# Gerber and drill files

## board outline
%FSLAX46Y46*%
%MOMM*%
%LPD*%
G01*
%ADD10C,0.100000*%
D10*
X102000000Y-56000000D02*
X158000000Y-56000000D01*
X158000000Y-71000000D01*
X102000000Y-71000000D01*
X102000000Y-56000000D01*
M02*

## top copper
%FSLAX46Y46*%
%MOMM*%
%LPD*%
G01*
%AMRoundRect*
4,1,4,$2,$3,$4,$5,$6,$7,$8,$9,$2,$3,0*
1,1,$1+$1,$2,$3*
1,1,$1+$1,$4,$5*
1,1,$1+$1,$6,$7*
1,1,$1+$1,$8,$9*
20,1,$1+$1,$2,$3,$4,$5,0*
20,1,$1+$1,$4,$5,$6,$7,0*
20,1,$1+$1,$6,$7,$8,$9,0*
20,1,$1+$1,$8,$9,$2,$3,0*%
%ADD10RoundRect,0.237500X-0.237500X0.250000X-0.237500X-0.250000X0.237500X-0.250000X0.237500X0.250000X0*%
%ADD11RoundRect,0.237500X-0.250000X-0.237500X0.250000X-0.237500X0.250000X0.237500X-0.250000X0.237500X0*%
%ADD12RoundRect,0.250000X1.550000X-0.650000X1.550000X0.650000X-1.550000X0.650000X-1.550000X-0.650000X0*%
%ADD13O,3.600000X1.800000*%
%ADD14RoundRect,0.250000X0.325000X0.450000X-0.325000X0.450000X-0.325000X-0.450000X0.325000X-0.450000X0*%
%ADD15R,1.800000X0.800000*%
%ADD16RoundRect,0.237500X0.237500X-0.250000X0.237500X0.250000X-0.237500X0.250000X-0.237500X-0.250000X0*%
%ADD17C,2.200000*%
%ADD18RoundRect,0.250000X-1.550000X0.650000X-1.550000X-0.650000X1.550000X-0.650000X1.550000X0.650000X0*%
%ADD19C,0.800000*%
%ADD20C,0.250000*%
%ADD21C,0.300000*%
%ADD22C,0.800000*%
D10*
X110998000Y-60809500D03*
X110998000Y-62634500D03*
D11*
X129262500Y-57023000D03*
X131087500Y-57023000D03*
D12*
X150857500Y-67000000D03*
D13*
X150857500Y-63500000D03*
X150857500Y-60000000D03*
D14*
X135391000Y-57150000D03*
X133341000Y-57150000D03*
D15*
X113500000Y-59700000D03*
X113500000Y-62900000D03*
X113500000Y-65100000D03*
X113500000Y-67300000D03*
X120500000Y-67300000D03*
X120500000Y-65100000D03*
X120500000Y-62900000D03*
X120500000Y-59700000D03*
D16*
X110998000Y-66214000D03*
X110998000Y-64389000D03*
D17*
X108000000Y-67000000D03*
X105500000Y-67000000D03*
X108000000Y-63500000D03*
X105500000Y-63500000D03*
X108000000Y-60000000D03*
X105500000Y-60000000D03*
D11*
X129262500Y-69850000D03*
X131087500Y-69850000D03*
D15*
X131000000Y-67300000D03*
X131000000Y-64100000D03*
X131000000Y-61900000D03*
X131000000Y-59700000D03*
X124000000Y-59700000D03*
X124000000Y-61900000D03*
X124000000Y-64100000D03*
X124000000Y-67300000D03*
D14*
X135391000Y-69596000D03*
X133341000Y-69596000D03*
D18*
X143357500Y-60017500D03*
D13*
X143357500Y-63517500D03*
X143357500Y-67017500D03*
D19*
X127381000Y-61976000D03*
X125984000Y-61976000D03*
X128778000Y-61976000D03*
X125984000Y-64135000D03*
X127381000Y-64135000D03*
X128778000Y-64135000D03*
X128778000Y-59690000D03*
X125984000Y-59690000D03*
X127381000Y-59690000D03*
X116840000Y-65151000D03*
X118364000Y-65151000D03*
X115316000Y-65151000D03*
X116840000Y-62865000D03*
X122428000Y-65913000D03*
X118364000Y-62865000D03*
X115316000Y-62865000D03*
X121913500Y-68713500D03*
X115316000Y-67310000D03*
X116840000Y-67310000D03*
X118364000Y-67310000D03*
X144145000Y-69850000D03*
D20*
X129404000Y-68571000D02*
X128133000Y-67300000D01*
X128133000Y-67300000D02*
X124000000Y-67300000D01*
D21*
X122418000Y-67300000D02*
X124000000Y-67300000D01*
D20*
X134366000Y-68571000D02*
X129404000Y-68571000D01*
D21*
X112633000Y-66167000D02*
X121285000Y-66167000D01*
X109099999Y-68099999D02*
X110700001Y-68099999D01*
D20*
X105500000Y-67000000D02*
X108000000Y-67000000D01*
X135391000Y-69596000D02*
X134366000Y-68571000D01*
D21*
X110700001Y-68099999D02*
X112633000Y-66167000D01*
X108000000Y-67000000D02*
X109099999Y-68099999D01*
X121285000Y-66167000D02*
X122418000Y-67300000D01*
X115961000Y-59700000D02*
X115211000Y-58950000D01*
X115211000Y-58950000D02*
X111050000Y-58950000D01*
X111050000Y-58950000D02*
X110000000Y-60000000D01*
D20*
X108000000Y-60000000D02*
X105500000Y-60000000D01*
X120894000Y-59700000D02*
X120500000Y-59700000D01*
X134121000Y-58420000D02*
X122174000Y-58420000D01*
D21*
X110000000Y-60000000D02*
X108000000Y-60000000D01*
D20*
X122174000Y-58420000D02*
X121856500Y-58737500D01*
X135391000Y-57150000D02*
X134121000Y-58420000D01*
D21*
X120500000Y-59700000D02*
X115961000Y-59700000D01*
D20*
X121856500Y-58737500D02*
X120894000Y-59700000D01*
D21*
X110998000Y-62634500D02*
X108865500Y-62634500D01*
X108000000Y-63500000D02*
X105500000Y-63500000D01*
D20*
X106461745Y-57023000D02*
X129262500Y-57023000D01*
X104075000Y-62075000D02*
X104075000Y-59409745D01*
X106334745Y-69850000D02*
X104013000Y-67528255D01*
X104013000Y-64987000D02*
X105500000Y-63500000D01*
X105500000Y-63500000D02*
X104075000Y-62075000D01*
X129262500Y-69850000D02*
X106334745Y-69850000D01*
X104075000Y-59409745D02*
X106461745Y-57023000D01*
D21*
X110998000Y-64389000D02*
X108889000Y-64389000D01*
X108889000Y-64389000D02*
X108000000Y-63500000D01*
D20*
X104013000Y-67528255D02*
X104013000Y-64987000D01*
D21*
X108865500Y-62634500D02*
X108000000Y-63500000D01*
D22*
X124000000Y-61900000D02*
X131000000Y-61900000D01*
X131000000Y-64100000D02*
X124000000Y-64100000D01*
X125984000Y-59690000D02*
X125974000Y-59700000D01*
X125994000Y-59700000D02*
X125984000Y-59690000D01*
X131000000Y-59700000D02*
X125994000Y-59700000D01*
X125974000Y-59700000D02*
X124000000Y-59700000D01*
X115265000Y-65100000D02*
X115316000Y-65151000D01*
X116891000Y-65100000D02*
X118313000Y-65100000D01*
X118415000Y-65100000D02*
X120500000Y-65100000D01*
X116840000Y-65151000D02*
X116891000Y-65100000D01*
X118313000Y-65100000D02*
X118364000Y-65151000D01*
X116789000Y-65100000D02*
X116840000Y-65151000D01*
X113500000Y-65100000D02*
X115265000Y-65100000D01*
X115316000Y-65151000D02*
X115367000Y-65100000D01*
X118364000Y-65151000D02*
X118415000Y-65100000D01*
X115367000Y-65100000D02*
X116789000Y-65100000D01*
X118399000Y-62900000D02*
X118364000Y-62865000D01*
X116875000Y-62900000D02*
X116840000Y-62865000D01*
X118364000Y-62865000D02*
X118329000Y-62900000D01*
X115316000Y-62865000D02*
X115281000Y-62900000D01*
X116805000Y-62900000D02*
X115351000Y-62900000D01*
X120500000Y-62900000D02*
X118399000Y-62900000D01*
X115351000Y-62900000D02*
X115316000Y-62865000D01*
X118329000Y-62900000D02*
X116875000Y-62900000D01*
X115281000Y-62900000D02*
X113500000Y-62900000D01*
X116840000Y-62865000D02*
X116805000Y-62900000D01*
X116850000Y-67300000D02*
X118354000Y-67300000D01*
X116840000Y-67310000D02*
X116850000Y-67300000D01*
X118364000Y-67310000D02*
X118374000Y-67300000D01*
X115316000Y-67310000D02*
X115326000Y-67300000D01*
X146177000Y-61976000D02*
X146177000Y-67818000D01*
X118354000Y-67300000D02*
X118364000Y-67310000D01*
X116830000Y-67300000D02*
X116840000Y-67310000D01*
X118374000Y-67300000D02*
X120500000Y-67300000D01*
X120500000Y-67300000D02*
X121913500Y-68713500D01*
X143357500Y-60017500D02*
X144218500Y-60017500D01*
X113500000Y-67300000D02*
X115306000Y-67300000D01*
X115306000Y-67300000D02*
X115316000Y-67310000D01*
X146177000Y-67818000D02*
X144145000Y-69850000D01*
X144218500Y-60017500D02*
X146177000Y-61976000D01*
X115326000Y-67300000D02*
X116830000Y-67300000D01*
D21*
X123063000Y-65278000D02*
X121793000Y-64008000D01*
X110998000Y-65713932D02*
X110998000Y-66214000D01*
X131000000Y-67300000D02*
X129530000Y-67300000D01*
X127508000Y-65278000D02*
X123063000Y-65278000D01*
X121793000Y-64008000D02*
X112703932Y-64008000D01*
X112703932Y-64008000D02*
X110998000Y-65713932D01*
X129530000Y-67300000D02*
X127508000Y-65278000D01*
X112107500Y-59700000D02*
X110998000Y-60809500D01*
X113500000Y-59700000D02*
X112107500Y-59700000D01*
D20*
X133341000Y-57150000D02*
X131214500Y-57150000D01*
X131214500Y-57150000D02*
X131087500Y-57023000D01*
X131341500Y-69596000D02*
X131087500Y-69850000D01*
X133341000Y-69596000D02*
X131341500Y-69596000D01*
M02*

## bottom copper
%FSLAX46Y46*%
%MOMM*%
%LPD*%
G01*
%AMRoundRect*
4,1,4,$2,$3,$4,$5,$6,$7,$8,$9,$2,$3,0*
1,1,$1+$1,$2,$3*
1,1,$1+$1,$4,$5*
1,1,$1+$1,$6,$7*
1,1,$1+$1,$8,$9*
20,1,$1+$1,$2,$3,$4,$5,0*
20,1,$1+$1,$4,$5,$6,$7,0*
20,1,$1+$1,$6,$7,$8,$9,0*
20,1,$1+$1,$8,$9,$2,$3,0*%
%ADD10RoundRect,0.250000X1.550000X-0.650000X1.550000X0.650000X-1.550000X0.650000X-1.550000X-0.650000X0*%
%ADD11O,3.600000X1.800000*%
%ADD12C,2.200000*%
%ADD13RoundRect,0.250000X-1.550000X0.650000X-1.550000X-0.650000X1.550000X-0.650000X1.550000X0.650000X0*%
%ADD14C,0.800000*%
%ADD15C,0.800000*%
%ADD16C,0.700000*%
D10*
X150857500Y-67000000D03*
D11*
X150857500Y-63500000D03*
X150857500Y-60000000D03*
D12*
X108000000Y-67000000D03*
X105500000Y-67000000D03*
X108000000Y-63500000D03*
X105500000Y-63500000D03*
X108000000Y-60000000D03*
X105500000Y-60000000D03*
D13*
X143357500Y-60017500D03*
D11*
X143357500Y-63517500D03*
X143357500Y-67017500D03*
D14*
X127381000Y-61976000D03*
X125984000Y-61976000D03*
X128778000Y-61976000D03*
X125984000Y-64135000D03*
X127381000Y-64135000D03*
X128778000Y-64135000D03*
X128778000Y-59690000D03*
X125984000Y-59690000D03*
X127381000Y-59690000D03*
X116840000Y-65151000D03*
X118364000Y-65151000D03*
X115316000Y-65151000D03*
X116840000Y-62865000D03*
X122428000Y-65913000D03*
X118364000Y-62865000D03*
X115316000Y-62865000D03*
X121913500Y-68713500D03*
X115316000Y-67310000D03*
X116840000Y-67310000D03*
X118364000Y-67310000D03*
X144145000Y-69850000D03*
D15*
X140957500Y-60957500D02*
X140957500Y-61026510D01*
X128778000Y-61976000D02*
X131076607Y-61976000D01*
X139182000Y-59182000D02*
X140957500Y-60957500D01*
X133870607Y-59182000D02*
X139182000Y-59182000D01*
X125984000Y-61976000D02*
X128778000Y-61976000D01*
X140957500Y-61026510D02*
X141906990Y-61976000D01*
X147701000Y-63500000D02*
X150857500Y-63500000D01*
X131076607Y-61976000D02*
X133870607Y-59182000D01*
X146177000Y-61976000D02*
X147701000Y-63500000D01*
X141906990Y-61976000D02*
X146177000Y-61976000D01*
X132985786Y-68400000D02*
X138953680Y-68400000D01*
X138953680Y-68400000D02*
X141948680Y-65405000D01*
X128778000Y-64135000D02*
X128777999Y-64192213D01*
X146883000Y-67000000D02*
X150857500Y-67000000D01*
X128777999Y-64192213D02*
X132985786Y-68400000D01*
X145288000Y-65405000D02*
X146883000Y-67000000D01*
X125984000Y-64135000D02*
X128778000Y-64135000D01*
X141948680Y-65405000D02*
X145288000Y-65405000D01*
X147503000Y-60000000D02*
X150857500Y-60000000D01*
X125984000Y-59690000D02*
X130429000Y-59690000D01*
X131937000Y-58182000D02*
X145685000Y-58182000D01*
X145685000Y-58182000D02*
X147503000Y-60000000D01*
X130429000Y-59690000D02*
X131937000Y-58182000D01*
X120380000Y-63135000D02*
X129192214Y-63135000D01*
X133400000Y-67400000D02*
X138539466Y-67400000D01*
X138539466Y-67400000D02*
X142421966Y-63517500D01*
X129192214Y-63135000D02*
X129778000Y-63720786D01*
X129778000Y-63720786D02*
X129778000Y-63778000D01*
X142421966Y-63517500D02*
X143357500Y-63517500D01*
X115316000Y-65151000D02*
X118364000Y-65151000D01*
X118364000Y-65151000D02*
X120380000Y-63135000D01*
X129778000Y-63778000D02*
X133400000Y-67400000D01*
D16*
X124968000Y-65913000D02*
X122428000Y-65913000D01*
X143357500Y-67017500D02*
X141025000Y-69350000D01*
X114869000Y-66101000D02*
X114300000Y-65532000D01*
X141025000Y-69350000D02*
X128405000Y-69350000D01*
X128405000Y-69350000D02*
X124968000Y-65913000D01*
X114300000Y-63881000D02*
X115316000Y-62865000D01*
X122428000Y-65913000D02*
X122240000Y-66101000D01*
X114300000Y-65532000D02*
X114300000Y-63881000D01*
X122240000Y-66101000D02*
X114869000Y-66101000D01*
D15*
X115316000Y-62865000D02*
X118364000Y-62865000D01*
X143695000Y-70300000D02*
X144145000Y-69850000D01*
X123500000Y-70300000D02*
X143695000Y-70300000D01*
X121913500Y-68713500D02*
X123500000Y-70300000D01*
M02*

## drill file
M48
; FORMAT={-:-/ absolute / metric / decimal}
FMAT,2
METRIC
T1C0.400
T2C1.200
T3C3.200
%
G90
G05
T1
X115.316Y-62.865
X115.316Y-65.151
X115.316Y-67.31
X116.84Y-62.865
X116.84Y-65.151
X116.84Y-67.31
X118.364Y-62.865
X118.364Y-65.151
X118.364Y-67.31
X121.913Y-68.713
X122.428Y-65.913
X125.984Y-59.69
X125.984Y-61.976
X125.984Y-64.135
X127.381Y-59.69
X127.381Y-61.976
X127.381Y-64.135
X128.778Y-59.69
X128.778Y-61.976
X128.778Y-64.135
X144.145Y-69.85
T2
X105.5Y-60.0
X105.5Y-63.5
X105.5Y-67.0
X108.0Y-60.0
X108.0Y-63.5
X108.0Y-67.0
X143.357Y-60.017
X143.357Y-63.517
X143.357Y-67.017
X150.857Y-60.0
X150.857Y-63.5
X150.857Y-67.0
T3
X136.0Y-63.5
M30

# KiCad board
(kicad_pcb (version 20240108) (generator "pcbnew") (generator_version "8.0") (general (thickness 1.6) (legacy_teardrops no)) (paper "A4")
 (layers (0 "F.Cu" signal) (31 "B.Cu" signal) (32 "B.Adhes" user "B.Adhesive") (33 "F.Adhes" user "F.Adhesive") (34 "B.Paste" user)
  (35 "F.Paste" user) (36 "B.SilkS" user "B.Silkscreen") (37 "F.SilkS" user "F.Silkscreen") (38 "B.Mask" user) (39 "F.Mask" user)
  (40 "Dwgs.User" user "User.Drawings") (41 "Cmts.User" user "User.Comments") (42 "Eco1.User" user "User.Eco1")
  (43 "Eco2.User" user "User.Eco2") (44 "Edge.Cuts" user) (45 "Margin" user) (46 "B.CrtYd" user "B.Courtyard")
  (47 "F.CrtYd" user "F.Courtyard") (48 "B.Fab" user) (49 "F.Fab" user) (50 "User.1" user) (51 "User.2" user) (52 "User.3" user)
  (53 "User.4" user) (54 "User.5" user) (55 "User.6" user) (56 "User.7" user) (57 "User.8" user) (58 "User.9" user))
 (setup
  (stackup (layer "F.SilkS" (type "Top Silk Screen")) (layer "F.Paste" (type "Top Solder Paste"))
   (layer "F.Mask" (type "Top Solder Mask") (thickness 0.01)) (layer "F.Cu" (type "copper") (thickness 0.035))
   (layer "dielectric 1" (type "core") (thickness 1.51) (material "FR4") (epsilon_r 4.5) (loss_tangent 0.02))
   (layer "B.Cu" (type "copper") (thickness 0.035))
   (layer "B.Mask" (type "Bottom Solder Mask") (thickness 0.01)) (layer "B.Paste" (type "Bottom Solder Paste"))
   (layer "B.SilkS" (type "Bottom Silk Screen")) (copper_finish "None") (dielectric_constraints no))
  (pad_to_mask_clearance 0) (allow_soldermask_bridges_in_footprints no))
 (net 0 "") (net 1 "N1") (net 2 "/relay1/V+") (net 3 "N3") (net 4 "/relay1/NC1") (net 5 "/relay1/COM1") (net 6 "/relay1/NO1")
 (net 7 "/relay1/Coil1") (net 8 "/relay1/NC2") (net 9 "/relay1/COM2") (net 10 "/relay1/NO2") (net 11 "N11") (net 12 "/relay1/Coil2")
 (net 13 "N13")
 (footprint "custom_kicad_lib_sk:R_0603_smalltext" (layer "F.Cu") (at 110.998 61.722 -90)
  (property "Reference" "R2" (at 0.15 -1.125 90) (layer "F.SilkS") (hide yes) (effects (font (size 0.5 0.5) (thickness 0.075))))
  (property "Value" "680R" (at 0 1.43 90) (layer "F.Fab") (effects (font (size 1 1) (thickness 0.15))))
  (pad "1" smd roundrect (at -0.9125 0 270) (size 0.975 0.95) (layers "F.Cu" "F.Paste" "F.Mask") (roundrect_rratio 0.25) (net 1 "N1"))
  (pad "2" smd roundrect (at 0.9125 0 270) (size 0.975 0.95) (layers "F.Cu" "F.Paste" "F.Mask") (roundrect_rratio 0.25) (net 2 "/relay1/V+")))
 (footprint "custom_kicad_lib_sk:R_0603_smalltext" (layer "F.Cu") (at 130.175 57.023)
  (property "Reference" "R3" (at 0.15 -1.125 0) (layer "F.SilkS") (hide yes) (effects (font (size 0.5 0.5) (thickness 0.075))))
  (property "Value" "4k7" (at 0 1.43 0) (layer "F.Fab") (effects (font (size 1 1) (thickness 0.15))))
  (pad "1" smd roundrect (at -0.9125 0) (size 0.975 0.95) (layers "F.Cu" "F.Paste" "F.Mask") (roundrect_rratio 0.25) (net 2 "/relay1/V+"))
  (pad "2" smd roundrect (at 0.9125 0) (size 0.975 0.95) (layers "F.Cu" "F.Paste" "F.Mask") (roundrect_rratio 0.25) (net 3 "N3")))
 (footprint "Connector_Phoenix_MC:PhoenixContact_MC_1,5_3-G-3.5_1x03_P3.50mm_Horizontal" (layer "F.Cu") (at 150.8575 67 90)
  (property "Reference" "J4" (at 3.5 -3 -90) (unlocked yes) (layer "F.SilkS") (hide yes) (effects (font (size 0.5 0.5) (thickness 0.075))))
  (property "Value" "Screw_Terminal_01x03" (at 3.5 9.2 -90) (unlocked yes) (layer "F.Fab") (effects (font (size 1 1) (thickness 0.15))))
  (pad "1" thru_hole roundrect (at 0 0 90) (size 1.8 3.6) (drill 1.2) (layers "*.Cu" "*.Mask") (remove_unused_layers no)
   (roundrect_rratio 0.138889) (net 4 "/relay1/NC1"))
  (pad "2" thru_hole oval (at 3.5 0 90) (size 1.8 3.6) (drill 1.2) (layers "*.Cu" "*.Mask") (remove_unused_layers no) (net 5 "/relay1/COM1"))
  (pad "3" thru_hole oval (at 7 0 90) (size 1.8 3.6) (drill 1.2) (layers "*.Cu" "*.Mask") (remove_unused_layers no) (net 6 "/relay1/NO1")))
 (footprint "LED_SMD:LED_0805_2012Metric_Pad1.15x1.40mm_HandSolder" (layer "F.Cu") (at 134.366 57.15 180)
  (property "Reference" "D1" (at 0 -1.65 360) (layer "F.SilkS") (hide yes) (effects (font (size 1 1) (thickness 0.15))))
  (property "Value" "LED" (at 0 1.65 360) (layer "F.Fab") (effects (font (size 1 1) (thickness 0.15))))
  (pad "1" smd roundrect (at -1.025 0 180) (size 1.15 1.4) (layers "F.Cu" "F.Paste" "F.Mask") (roundrect_rratio 0.217391)
   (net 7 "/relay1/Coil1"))
  (pad "2" smd roundrect (at 1.025 0 180) (size 1.15 1.4) (layers "F.Cu" "F.Paste" "F.Mask") (roundrect_rratio 0.217391) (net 3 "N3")))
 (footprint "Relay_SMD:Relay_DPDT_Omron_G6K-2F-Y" (layer "F.Cu") (at 117 63.5)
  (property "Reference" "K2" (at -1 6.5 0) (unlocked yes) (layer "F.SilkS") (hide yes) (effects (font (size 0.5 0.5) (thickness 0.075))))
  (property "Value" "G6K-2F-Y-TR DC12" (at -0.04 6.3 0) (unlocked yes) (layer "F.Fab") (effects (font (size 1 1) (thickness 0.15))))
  (pad "1" smd rect (at -3.5 -3.8) (size 1.8 0.8) (layers "F.Cu" "F.Paste" "F.Mask") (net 1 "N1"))
  (pad "2" smd rect (at -3.5 -0.6) (size 1.8 0.8) (layers "F.Cu" "F.Paste" "F.Mask") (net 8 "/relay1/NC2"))
  (pad "3" smd rect (at -3.5 1.6) (size 1.8 0.8) (layers "F.Cu" "F.Paste" "F.Mask") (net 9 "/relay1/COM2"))
  (pad "4" smd rect (at -3.5 3.8) (size 1.8 0.8) (layers "F.Cu" "F.Paste" "F.Mask") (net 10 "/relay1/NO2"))
  (pad "5" smd rect (at 3.5 3.8) (size 1.8 0.8) (layers "F.Cu" "F.Paste" "F.Mask") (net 10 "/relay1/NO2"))
  (pad "6" smd rect (at 3.5 1.6) (size 1.8 0.8) (layers "F.Cu" "F.Paste" "F.Mask") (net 9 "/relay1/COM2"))
  (pad "7" smd rect (at 3.5 -0.6) (size 1.8 0.8) (layers "F.Cu" "F.Paste" "F.Mask") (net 8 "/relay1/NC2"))
  (pad "8" smd rect (at 3.5 -3.8) (size 1.8 0.8) (layers "F.Cu" "F.Paste" "F.Mask") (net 7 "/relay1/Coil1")))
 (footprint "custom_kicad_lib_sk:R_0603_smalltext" (layer "F.Cu") (at 110.998 65.3015 90)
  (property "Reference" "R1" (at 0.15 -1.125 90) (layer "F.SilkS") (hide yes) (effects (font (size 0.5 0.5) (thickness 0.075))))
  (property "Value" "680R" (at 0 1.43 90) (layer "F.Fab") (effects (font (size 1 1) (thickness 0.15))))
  (pad "1" smd roundrect (at -0.9125 0 90) (size 0.975 0.95) (layers "F.Cu" "F.Paste" "F.Mask") (roundrect_rratio 0.25) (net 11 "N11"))
  (pad "2" smd roundrect (at 0.9125 0 90) (size 0.975 0.95) (layers "F.Cu" "F.Paste" "F.Mask") (roundrect_rratio 0.25) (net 2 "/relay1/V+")))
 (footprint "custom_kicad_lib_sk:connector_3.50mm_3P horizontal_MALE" (layer "F.Cu") (at 108 63.5 -90)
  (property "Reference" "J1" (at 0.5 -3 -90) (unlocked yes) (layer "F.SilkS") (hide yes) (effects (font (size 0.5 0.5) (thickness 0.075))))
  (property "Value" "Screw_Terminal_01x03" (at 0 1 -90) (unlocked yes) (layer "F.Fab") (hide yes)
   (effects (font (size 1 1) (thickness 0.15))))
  (pad "1" thru_hole circle (at 3.5 0 270) (size 2.2 2.2) (drill 1.2) (layers "*.Cu" "*.Mask") (remove_unused_layers no)
   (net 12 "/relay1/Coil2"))
  (pad "1" thru_hole circle (at 3.5 2.5 270) (size 2.2 2.2) (drill 1.2) (layers "*.Cu" "*.Mask") (remove_unused_layers no)
   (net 12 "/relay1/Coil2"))
  (pad "2" thru_hole circle (at 0 0 270) (size 2.2 2.2) (drill 1.2) (layers "*.Cu" "*.Mask") (remove_unused_layers no) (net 2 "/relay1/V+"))
  (pad "2" thru_hole circle (at 0 2.5 270) (size 2.2 2.2) (drill 1.2) (layers "*.Cu" "*.Mask") (remove_unused_layers no)
   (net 2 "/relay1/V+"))
  (pad "3" thru_hole circle (at -3.5 0 270) (size 2.2 2.2) (drill 1.2) (layers "*.Cu" "*.Mask") (remove_unused_layers no)
   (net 7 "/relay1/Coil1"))
  (pad "3" thru_hole circle (at -3.5 2.5 270) (size 2.2 2.2) (drill 1.2) (layers "*.Cu" "*.Mask") (remove_unused_layers no)
   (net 7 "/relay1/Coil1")))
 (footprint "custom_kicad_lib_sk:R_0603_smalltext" (layer "F.Cu") (at 130.175 69.85)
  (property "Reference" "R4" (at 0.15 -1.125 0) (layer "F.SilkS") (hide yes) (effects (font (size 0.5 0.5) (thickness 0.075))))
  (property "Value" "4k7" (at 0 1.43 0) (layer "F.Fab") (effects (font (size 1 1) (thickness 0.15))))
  (pad "1" smd roundrect (at -0.9125 0) (size 0.975 0.95) (layers "F.Cu" "F.Paste" "F.Mask") (roundrect_rratio 0.25) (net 2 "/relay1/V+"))
  (pad "2" smd roundrect (at 0.9125 0) (size 0.975 0.95) (layers "F.Cu" "F.Paste" "F.Mask") (roundrect_rratio 0.25) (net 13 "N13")))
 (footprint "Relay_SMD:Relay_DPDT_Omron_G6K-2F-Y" (layer "F.Cu") (at 127.5 63.5 180)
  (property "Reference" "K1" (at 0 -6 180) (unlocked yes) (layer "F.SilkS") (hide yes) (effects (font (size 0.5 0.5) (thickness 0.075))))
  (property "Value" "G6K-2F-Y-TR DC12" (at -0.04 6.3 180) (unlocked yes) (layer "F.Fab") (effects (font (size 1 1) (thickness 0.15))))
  (pad "1" smd rect (at -3.5 -3.8 180) (size 1.8 0.8) (layers "F.Cu" "F.Paste" "F.Mask") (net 11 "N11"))
  (pad "2" smd rect (at -3.5 -0.6 180) (size 1.8 0.8) (layers "F.Cu" "F.Paste" "F.Mask") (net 4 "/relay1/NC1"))
  (pad "3" smd rect (at -3.5 1.6 180) (size 1.8 0.8) (layers "F.Cu" "F.Paste" "F.Mask") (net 5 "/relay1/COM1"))
  (pad "4" smd rect (at -3.5 3.8 180) (size 1.8 0.8) (layers "F.Cu" "F.Paste" "F.Mask") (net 6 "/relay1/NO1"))
  (pad "5" smd rect (at 3.5 3.8 180) (size 1.8 0.8) (layers "F.Cu" "F.Paste" "F.Mask") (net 6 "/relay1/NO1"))
  (pad "6" smd rect (at 3.5 1.6 180) (size 1.8 0.8) (layers "F.Cu" "F.Paste" "F.Mask") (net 5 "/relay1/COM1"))
  (pad "7" smd rect (at 3.5 -0.6 180) (size 1.8 0.8) (layers "F.Cu" "F.Paste" "F.Mask") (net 4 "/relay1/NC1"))
  (pad "8" smd rect (at 3.5 -3.8 180) (size 1.8 0.8) (layers "F.Cu" "F.Paste" "F.Mask") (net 12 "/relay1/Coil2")))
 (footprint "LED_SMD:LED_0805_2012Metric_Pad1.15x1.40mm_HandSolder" (layer "F.Cu") (at 134.366 69.596 180)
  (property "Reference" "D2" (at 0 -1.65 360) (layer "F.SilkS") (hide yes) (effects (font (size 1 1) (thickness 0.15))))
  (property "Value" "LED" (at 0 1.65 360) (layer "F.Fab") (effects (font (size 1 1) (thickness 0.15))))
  (pad "1" smd roundrect (at -1.025 0 180) (size 1.15 1.4) (layers "F.Cu" "F.Paste" "F.Mask") (roundrect_rratio 0.217391)
   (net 12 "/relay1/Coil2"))
  (pad "2" smd roundrect (at 1.025 0 180) (size 1.15 1.4) (layers "F.Cu" "F.Paste" "F.Mask") (roundrect_rratio 0.217391) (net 13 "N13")))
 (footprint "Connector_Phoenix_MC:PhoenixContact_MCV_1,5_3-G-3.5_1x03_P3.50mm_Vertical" (layer "F.Cu") (at 143.3575 60.0175 -90)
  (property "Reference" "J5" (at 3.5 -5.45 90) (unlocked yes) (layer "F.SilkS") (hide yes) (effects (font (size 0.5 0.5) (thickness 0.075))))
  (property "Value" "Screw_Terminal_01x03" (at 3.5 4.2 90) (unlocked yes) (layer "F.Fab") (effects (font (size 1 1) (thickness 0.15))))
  (pad "1" thru_hole roundrect (at 0 0 270) (size 1.8 3.6) (drill 1.2) (layers "*.Cu" "*.Mask") (remove_unused_layers no)
   (roundrect_rratio 0.138889) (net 10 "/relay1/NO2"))
  (pad "2" thru_hole oval (at 3.5 0 270) (size 1.8 3.6) (drill 1.2) (layers "*.Cu" "*.Mask") (remove_unused_layers no)
   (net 9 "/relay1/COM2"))
  (pad "3" thru_hole oval (at 7 0 270) (size 1.8 3.6) (drill 1.2) (layers "*.Cu" "*.Mask") (remove_unused_layers no) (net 8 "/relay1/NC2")))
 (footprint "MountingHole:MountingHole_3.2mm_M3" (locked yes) (layer "F.Cu") (at 136 63.5)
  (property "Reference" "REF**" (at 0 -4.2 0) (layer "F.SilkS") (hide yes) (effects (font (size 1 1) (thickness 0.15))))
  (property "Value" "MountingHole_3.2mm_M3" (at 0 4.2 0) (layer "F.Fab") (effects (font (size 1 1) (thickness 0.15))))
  (pad "" np_thru_hole circle (at 0 0) (size 3.2 3.2) (drill 3.2) (layers "*.Cu" "*.Mask")))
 (gr_rect (start 102 56) (end 158 71) (stroke (width 0.1) (type default)) (fill none) (layer "Edge.Cuts"))
 (segment (start 129.404 68.571) (end 128.133 67.3) (width 0.25) (layer "F.Cu") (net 12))
 (segment (start 128.133 67.3) (end 124 67.3) (width 0.25) (layer "F.Cu") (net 12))
 (segment (start 122.418 67.3) (end 124 67.3) (width 0.3) (layer "F.Cu") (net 12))
 (segment (start 134.366 68.571) (end 129.404 68.571) (width 0.25) (layer "F.Cu") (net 12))
 (segment (start 112.633 66.167) (end 121.285 66.167) (width 0.3) (layer "F.Cu") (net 12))
 (segment (start 109.099999 68.099999) (end 110.700001 68.099999) (width 0.3) (layer "F.Cu") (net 12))
 (segment (start 105.5 67) (end 108 67) (width 0.25) (layer "F.Cu") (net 12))
 (segment (start 135.391 69.596) (end 134.366 68.571) (width 0.25) (layer "F.Cu") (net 12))
 (segment (start 110.700001 68.099999) (end 112.633 66.167) (width 0.3) (layer "F.Cu") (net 12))
 (segment (start 108 67) (end 109.099999 68.099999) (width 0.3) (layer "F.Cu") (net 12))
 (segment (start 121.285 66.167) (end 122.418 67.3) (width 0.3) (layer "F.Cu") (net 12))
 (segment (start 115.961 59.7) (end 115.211 58.95) (width 0.3) (layer "F.Cu") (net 7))
 (segment (start 115.211 58.95) (end 111.05 58.95) (width 0.3) (layer "F.Cu") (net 7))
 (segment (start 111.05 58.95) (end 110 60) (width 0.3) (layer "F.Cu") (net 7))
 (segment (start 108 60) (end 105.5 60) (width 0.25) (layer "F.Cu") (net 7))
 (segment (start 120.894 59.7) (end 120.5 59.7) (width 0.25) (layer "F.Cu") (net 7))
 (segment (start 134.121 58.42) (end 122.174 58.42) (width 0.25) (layer "F.Cu") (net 7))
 (segment (start 110 60) (end 108 60) (width 0.3) (layer "F.Cu") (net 7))
 (segment (start 122.174 58.42) (end 121.8565 58.7375) (width 0.25) (layer "F.Cu") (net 7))
 (segment (start 135.391 57.15) (end 134.121 58.42) (width 0.25) (layer "F.Cu") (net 7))
 (segment (start 120.5 59.7) (end 115.961 59.7) (width 0.3) (layer "F.Cu") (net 7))
 (segment (start 121.8565 58.7375) (end 120.894 59.7) (width 0.25) (layer "F.Cu") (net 7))
 (segment (start 110.998 62.6345) (end 108.8655 62.6345) (width 0.3) (layer "F.Cu") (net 2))
 (segment (start 108 63.5) (end 105.5 63.5) (width 0.3) (layer "F.Cu") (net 2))
 (segment (start 106.461745 57.023) (end 129.2625 57.023) (width 0.25) (layer "F.Cu") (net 2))
 (segment (start 104.075 62.075) (end 104.075 59.409745) (width 0.25) (layer "F.Cu") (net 2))
 (segment (start 106.334745 69.85) (end 104.013 67.528255) (width 0.25) (layer "F.Cu") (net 2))
 (segment (start 104.013 64.987) (end 105.5 63.5) (width 0.25) (layer "F.Cu") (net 2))
 (segment (start 105.5 63.5) (end 104.075 62.075) (width 0.25) (layer "F.Cu") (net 2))
 (segment (start 129.2625 69.85) (end 106.334745 69.85) (width 0.25) (layer "F.Cu") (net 2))
 (segment (start 104.075 59.409745) (end 106.461745 57.023) (width 0.25) (layer "F.Cu") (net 2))
 (segment (start 110.998 64.389) (end 108.889 64.389) (width 0.3) (layer "F.Cu") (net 2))
 (segment (start 108.889 64.389) (end 108 63.5) (width 0.3) (layer "F.Cu") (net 2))
 (segment (start 104.013 67.528255) (end 104.013 64.987) (width 0.25) (layer "F.Cu") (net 2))
 (segment (start 108.8655 62.6345) (end 108 63.5) (width 0.3) (layer "F.Cu") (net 2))
 (segment (start 124 61.9) (end 131 61.9) (width 0.8) (layer "F.Cu") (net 5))
 (via (at 127.381 61.976) (size 0.8) (drill 0.4) (layers "F.Cu" "B.Cu") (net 5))
 (via (at 125.984 61.976) (size 0.8) (drill 0.4) (layers "F.Cu" "B.Cu") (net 5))
 (via (at 128.778 61.976) (size 0.8) (drill 0.4) (layers "F.Cu" "B.Cu") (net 5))
 (segment (start 140.9575 60.9575) (end 140.9575 61.02651) (width 0.8) (layer "B.Cu") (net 5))
 (segment (start 128.778 61.976) (end 131.076607 61.976) (width 0.8) (layer "B.Cu") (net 5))
 (segment (start 139.182 59.182) (end 140.9575 60.9575) (width 0.8) (layer "B.Cu") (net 5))
 (segment (start 133.870607 59.182) (end 139.182 59.182) (width 0.8) (layer "B.Cu") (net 5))
 (segment (start 125.984 61.976) (end 128.778 61.976) (width 0.8) (layer "B.Cu") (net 5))
 (segment (start 140.9575 61.02651) (end 141.90699 61.976) (width 0.8) (layer "B.Cu") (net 5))
 (segment (start 147.701 63.5) (end 150.8575 63.5) (width 0.8) (layer "B.Cu") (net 5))
 (segment (start 131.076607 61.976) (end 133.870607 59.182) (width 0.8) (layer "B.Cu") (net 5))
 (segment (start 146.177 61.976) (end 147.701 63.5) (width 0.8) (layer "B.Cu") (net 5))
 (segment (start 141.90699 61.976) (end 146.177 61.976) (width 0.8) (layer "B.Cu") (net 5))
 (segment (start 131 64.1) (end 124 64.1) (width 0.8) (layer "F.Cu") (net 4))
 (via (at 125.984 64.135) (size 0.8) (drill 0.4) (layers "F.Cu" "B.Cu") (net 4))
 (via (at 127.381 64.135) (size 0.8) (drill 0.4) (layers "F.Cu" "B.Cu") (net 4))
 (via (at 128.778 64.135) (size 0.8) (drill 0.4) (layers "F.Cu" "B.Cu") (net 4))
 (segment (start 132.985786 68.4) (end 138.95368 68.4) (width 0.8) (layer "B.Cu") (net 4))
 (segment (start 138.95368 68.4) (end 141.94868 65.405) (width 0.8) (layer "B.Cu") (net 4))
 (segment (start 128.778 64.135) (end 128.777999 64.192213) (width 0.8) (layer "B.Cu") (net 4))
 (segment (start 146.883 67) (end 150.8575 67) (width 0.8) (layer "B.Cu") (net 4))
 (segment (start 128.777999 64.192213) (end 132.985786 68.4) (width 0.8) (layer "B.Cu") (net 4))
 (segment (start 145.288 65.405) (end 146.883 67) (width 0.8) (layer "B.Cu") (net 4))
 (segment (start 125.984 64.135) (end 128.778 64.135) (width 0.8) (layer "B.Cu") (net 4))
 (segment (start 141.94868 65.405) (end 145.288 65.405) (width 0.8) (layer "B.Cu") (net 4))
 (segment (start 125.984 59.69) (end 125.974 59.7) (width 0.8) (layer "F.Cu") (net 6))
 (segment (start 125.994 59.7) (end 125.984 59.69) (width 0.8) (layer "F.Cu") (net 6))
 (segment (start 131 59.7) (end 125.994 59.7) (width 0.8) (layer "F.Cu") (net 6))
 (segment (start 125.974 59.7) (end 124 59.7) (width 0.8) (layer "F.Cu") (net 6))
 (via (at 128.778 59.69) (size 0.8) (drill 0.4) (layers "F.Cu" "B.Cu") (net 6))
 (via (at 125.984 59.69) (size 0.8) (drill 0.4) (layers "F.Cu" "B.Cu") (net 6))
 (via (at 127.381 59.69) (size 0.8) (drill 0.4) (layers "F.Cu" "B.Cu") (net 6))
 (segment (start 147.503 60) (end 150.8575 60) (width 0.8) (layer "B.Cu") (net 6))
 (segment (start 125.984 59.69) (end 130.429 59.69) (width 0.8) (layer "B.Cu") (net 6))
 (segment (start 131.937 58.182) (end 145.685 58.182) (width 0.8) (layer "B.Cu") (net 6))
 (segment (start 145.685 58.182) (end 147.503 60) (width 0.8) (layer "B.Cu") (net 6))
 (segment (start 130.429 59.69) (end 131.937 58.182) (width 0.8) (layer "B.Cu") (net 6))
 (segment (start 115.265 65.1) (end 115.316 65.151) (width 0.8) (layer "F.Cu") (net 9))
 (segment (start 116.891 65.1) (end 118.313 65.1) (width 0.8) (layer "F.Cu") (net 9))
 (segment (start 118.415 65.1) (end 120.5 65.1) (width 0.8) (layer "F.Cu") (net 9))
 (segment (start 116.84 65.151) (end 116.891 65.1) (width 0.8) (layer "F.Cu") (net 9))
 (segment (start 118.313 65.1) (end 118.364 65.151) (width 0.8) (layer "F.Cu") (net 9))
 (segment (start 116.789 65.1) (end 116.84 65.151) (width 0.8) (layer "F.Cu") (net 9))
 (segment (start 113.5 65.1) (end 115.265 65.1) (width 0.8) (layer "F.Cu") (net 9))
 (segment (start 115.316 65.151) (end 115.367 65.1) (width 0.8) (layer "F.Cu") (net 9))
 (segment (start 118.364 65.151) (end 118.415 65.1) (width 0.8) (layer "F.Cu") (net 9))
 (segment (start 115.367 65.1) (end 116.789 65.1) (width 0.8) (layer "F.Cu") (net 9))
 (via (at 116.84 65.151) (size 0.8) (drill 0.4) (layers "F.Cu" "B.Cu") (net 9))
 (via (at 118.364 65.151) (size 0.8) (drill 0.4) (layers "F.Cu" "B.Cu") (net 9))
 (via (at 115.316 65.151) (size 0.8) (drill 0.4) (layers "F.Cu" "B.Cu") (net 9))
 (segment (start 120.38 63.135) (end 129.192214 63.135) (width 0.8) (layer "B.Cu") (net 9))
 (segment (start 133.4 67.4) (end 138.539466 67.4) (width 0.8) (layer "B.Cu") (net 9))
 (segment (start 138.539466 67.4) (end 142.421966 63.5175) (width 0.8) (layer "B.Cu") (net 9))
 (segment (start 129.192214 63.135) (end 129.778 63.720786) (width 0.8) (layer "B.Cu") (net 9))
 (segment (start 129.778 63.720786) (end 129.778 63.778) (width 0.8) (layer "B.Cu") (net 9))
 (segment (start 142.421966 63.5175) (end 143.3575 63.5175) (width 0.8) (layer "B.Cu") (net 9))
 (segment (start 115.316 65.151) (end 118.364 65.151) (width 0.8) (layer "B.Cu") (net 9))
 (segment (start 118.364 65.151) (end 120.38 63.135) (width 0.8) (layer "B.Cu") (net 9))
 (segment (start 129.778 63.778) (end 133.4 67.4) (width 0.8) (layer "B.Cu") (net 9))
 (segment (start 118.399 62.9) (end 118.364 62.865) (width 0.8) (layer "F.Cu") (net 8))
 (segment (start 116.875 62.9) (end 116.84 62.865) (width 0.8) (layer "F.Cu") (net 8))
 (segment (start 118.364 62.865) (end 118.329 62.9) (width 0.8) (layer "F.Cu") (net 8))
 (segment (start 115.316 62.865) (end 115.281 62.9) (width 0.8) (layer "F.Cu") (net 8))
 (segment (start 116.805 62.9) (end 115.351 62.9) (width 0.8) (layer "F.Cu") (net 8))
 (segment (start 120.5 62.9) (end 118.399 62.9) (width 0.8) (layer "F.Cu") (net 8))
 (segment (start 115.351 62.9) (end 115.316 62.865) (width 0.8) (layer "F.Cu") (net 8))
 (segment (start 118.329 62.9) (end 116.875 62.9) (width 0.8) (layer "F.Cu") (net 8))
 (segment (start 115.281 62.9) (end 113.5 62.9) (width 0.8) (layer "F.Cu") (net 8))
 (segment (start 116.84 62.865) (end 116.805 62.9) (width 0.8) (layer "F.Cu") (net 8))
 (via (at 116.84 62.865) (size 0.8) (drill 0.4) (layers "F.Cu" "B.Cu") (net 8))
 (via (at 122.428 65.913) (size 0.8) (drill 0.4) (layers "F.Cu" "B.Cu") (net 8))
 (via (at 118.364 62.865) (size 0.8) (drill 0.4) (layers "F.Cu" "B.Cu") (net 8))
 (via (at 115.316 62.865) (size 0.8) (drill 0.4) (layers "F.Cu" "B.Cu") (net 8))
 (segment (start 124.968 65.913) (end 122.428 65.913) (width 0.7) (layer "B.Cu") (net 8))
 (segment (start 143.3575 67.0175) (end 141.025 69.35) (width 0.7) (layer "B.Cu") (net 8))
 (segment (start 114.869 66.101) (end 114.3 65.532) (width 0.7) (layer "B.Cu") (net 8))
 (segment (start 141.025 69.35) (end 128.405 69.35) (width 0.7) (layer "B.Cu") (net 8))
 (segment (start 128.405 69.35) (end 124.968 65.913) (width 0.7) (layer "B.Cu") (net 8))
 (segment (start 114.3 63.881) (end 115.316 62.865) (width 0.7) (layer "B.Cu") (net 8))
 (segment (start 122.428 65.913) (end 122.24 66.101) (width 0.7) (layer "B.Cu") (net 8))
 (segment (start 114.3 65.532) (end 114.3 63.881) (width 0.7) (layer "B.Cu") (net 8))
 (segment (start 122.24 66.101) (end 114.869 66.101) (width 0.7) (layer "B.Cu") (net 8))
 (segment (start 115.316 62.865) (end 118.364 62.865) (width 0.8) (layer "B.Cu") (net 8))
 (segment (start 116.85 67.3) (end 118.354 67.3) (width 0.8) (layer "F.Cu") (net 10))
 (segment (start 116.84 67.31) (end 116.85 67.3) (width 0.8) (layer "F.Cu") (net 10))
 (segment (start 118.364 67.31) (end 118.374 67.3) (width 0.8) (layer "F.Cu") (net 10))
 (segment (start 115.316 67.31) (end 115.326 67.3) (width 0.8) (layer "F.Cu") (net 10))
 (segment (start 146.177 61.976) (end 146.177 67.818) (width 0.8) (layer "F.Cu") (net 10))
 (segment (start 118.354 67.3) (end 118.364 67.31) (width 0.8) (layer "F.Cu") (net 10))
 (segment (start 116.83 67.3) (end 116.84 67.31) (width 0.8) (layer "F.Cu") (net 10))
 (segment (start 118.374 67.3) (end 120.5 67.3) (width 0.8) (layer "F.Cu") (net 10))
 (segment (start 120.5 67.3) (end 121.9135 68.7135) (width 0.8) (layer "F.Cu") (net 10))
 (segment (start 143.3575 60.0175) (end 144.2185 60.0175) (width 0.8) (layer "F.Cu") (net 10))
 (segment (start 113.5 67.3) (end 115.306 67.3) (width 0.8) (layer "F.Cu") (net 10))
 (segment (start 115.306 67.3) (end 115.316 67.31) (width 0.8) (layer "F.Cu") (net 10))
 (segment (start 146.177 67.818) (end 144.145 69.85) (width 0.8) (layer "F.Cu") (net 10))
 (segment (start 144.2185 60.0175) (end 146.177 61.976) (width 0.8) (layer "F.Cu") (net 10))
 (segment (start 115.326 67.3) (end 116.83 67.3) (width 0.8) (layer "F.Cu") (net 10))
 (via (at 121.9135 68.7135) (size 0.8) (drill 0.4) (layers "F.Cu" "B.Cu") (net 10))
 (via (at 115.316 67.31) (size 0.8) (drill 0.4) (layers "F.Cu" "B.Cu") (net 10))
 (via (at 116.84 67.31) (size 0.8) (drill 0.4) (layers "F.Cu" "B.Cu") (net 10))
 (via (at 118.364 67.31) (size 0.8) (drill 0.4) (layers "F.Cu" "B.Cu") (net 10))
 (via (at 144.145 69.85) (size 0.8) (drill 0.4) (layers "F.Cu" "B.Cu") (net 10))
 (segment (start 143.695 70.3) (end 144.145 69.85) (width 0.8) (layer "B.Cu") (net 10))
 (segment (start 123.5 70.3) (end 143.695 70.3) (width 0.8) (layer "B.Cu") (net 10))
 (segment (start 121.9135 68.7135) (end 123.5 70.3) (width 0.8) (layer "B.Cu") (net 10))
 (segment (start 123.063 65.278) (end 121.793 64.008) (width 0.3) (layer "F.Cu") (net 11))
 (segment (start 110.998 65.713932) (end 110.998 66.214) (width 0.3) (layer "F.Cu") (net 11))
 (segment (start 131 67.3) (end 129.53 67.3) (width 0.3) (layer "F.Cu") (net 11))
 (segment (start 127.508 65.278) (end 123.063 65.278) (width 0.3) (layer "F.Cu") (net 11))
 (segment (start 121.793 64.008) (end 112.703932 64.008) (width 0.3) (layer "F.Cu") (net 11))
 (segment (start 112.703932 64.008) (end 110.998 65.713932) (width 0.3) (layer "F.Cu") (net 11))
 (segment (start 129.53 67.3) (end 127.508 65.278) (width 0.3) (layer "F.Cu") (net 11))
 (segment (start 112.1075 59.7) (end 110.998 60.8095) (width 0.3) (layer "F.Cu") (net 1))
 (segment (start 113.5 59.7) (end 112.1075 59.7) (width 0.3) (layer "F.Cu") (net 1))
 (segment (start 133.341 57.15) (end 131.2145 57.15) (width 0.25) (layer "F.Cu") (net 3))
 (segment (start 131.2145 57.15) (end 131.0875 57.023) (width 0.25) (layer "F.Cu") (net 3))
 (segment (start 131.3415 69.596) (end 131.0875 69.85) (width 0.25) (layer "F.Cu") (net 13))
 (segment (start 133.341 69.596) (end 131.3415 69.596) (width 0.25) (layer "F.Cu") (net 13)))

